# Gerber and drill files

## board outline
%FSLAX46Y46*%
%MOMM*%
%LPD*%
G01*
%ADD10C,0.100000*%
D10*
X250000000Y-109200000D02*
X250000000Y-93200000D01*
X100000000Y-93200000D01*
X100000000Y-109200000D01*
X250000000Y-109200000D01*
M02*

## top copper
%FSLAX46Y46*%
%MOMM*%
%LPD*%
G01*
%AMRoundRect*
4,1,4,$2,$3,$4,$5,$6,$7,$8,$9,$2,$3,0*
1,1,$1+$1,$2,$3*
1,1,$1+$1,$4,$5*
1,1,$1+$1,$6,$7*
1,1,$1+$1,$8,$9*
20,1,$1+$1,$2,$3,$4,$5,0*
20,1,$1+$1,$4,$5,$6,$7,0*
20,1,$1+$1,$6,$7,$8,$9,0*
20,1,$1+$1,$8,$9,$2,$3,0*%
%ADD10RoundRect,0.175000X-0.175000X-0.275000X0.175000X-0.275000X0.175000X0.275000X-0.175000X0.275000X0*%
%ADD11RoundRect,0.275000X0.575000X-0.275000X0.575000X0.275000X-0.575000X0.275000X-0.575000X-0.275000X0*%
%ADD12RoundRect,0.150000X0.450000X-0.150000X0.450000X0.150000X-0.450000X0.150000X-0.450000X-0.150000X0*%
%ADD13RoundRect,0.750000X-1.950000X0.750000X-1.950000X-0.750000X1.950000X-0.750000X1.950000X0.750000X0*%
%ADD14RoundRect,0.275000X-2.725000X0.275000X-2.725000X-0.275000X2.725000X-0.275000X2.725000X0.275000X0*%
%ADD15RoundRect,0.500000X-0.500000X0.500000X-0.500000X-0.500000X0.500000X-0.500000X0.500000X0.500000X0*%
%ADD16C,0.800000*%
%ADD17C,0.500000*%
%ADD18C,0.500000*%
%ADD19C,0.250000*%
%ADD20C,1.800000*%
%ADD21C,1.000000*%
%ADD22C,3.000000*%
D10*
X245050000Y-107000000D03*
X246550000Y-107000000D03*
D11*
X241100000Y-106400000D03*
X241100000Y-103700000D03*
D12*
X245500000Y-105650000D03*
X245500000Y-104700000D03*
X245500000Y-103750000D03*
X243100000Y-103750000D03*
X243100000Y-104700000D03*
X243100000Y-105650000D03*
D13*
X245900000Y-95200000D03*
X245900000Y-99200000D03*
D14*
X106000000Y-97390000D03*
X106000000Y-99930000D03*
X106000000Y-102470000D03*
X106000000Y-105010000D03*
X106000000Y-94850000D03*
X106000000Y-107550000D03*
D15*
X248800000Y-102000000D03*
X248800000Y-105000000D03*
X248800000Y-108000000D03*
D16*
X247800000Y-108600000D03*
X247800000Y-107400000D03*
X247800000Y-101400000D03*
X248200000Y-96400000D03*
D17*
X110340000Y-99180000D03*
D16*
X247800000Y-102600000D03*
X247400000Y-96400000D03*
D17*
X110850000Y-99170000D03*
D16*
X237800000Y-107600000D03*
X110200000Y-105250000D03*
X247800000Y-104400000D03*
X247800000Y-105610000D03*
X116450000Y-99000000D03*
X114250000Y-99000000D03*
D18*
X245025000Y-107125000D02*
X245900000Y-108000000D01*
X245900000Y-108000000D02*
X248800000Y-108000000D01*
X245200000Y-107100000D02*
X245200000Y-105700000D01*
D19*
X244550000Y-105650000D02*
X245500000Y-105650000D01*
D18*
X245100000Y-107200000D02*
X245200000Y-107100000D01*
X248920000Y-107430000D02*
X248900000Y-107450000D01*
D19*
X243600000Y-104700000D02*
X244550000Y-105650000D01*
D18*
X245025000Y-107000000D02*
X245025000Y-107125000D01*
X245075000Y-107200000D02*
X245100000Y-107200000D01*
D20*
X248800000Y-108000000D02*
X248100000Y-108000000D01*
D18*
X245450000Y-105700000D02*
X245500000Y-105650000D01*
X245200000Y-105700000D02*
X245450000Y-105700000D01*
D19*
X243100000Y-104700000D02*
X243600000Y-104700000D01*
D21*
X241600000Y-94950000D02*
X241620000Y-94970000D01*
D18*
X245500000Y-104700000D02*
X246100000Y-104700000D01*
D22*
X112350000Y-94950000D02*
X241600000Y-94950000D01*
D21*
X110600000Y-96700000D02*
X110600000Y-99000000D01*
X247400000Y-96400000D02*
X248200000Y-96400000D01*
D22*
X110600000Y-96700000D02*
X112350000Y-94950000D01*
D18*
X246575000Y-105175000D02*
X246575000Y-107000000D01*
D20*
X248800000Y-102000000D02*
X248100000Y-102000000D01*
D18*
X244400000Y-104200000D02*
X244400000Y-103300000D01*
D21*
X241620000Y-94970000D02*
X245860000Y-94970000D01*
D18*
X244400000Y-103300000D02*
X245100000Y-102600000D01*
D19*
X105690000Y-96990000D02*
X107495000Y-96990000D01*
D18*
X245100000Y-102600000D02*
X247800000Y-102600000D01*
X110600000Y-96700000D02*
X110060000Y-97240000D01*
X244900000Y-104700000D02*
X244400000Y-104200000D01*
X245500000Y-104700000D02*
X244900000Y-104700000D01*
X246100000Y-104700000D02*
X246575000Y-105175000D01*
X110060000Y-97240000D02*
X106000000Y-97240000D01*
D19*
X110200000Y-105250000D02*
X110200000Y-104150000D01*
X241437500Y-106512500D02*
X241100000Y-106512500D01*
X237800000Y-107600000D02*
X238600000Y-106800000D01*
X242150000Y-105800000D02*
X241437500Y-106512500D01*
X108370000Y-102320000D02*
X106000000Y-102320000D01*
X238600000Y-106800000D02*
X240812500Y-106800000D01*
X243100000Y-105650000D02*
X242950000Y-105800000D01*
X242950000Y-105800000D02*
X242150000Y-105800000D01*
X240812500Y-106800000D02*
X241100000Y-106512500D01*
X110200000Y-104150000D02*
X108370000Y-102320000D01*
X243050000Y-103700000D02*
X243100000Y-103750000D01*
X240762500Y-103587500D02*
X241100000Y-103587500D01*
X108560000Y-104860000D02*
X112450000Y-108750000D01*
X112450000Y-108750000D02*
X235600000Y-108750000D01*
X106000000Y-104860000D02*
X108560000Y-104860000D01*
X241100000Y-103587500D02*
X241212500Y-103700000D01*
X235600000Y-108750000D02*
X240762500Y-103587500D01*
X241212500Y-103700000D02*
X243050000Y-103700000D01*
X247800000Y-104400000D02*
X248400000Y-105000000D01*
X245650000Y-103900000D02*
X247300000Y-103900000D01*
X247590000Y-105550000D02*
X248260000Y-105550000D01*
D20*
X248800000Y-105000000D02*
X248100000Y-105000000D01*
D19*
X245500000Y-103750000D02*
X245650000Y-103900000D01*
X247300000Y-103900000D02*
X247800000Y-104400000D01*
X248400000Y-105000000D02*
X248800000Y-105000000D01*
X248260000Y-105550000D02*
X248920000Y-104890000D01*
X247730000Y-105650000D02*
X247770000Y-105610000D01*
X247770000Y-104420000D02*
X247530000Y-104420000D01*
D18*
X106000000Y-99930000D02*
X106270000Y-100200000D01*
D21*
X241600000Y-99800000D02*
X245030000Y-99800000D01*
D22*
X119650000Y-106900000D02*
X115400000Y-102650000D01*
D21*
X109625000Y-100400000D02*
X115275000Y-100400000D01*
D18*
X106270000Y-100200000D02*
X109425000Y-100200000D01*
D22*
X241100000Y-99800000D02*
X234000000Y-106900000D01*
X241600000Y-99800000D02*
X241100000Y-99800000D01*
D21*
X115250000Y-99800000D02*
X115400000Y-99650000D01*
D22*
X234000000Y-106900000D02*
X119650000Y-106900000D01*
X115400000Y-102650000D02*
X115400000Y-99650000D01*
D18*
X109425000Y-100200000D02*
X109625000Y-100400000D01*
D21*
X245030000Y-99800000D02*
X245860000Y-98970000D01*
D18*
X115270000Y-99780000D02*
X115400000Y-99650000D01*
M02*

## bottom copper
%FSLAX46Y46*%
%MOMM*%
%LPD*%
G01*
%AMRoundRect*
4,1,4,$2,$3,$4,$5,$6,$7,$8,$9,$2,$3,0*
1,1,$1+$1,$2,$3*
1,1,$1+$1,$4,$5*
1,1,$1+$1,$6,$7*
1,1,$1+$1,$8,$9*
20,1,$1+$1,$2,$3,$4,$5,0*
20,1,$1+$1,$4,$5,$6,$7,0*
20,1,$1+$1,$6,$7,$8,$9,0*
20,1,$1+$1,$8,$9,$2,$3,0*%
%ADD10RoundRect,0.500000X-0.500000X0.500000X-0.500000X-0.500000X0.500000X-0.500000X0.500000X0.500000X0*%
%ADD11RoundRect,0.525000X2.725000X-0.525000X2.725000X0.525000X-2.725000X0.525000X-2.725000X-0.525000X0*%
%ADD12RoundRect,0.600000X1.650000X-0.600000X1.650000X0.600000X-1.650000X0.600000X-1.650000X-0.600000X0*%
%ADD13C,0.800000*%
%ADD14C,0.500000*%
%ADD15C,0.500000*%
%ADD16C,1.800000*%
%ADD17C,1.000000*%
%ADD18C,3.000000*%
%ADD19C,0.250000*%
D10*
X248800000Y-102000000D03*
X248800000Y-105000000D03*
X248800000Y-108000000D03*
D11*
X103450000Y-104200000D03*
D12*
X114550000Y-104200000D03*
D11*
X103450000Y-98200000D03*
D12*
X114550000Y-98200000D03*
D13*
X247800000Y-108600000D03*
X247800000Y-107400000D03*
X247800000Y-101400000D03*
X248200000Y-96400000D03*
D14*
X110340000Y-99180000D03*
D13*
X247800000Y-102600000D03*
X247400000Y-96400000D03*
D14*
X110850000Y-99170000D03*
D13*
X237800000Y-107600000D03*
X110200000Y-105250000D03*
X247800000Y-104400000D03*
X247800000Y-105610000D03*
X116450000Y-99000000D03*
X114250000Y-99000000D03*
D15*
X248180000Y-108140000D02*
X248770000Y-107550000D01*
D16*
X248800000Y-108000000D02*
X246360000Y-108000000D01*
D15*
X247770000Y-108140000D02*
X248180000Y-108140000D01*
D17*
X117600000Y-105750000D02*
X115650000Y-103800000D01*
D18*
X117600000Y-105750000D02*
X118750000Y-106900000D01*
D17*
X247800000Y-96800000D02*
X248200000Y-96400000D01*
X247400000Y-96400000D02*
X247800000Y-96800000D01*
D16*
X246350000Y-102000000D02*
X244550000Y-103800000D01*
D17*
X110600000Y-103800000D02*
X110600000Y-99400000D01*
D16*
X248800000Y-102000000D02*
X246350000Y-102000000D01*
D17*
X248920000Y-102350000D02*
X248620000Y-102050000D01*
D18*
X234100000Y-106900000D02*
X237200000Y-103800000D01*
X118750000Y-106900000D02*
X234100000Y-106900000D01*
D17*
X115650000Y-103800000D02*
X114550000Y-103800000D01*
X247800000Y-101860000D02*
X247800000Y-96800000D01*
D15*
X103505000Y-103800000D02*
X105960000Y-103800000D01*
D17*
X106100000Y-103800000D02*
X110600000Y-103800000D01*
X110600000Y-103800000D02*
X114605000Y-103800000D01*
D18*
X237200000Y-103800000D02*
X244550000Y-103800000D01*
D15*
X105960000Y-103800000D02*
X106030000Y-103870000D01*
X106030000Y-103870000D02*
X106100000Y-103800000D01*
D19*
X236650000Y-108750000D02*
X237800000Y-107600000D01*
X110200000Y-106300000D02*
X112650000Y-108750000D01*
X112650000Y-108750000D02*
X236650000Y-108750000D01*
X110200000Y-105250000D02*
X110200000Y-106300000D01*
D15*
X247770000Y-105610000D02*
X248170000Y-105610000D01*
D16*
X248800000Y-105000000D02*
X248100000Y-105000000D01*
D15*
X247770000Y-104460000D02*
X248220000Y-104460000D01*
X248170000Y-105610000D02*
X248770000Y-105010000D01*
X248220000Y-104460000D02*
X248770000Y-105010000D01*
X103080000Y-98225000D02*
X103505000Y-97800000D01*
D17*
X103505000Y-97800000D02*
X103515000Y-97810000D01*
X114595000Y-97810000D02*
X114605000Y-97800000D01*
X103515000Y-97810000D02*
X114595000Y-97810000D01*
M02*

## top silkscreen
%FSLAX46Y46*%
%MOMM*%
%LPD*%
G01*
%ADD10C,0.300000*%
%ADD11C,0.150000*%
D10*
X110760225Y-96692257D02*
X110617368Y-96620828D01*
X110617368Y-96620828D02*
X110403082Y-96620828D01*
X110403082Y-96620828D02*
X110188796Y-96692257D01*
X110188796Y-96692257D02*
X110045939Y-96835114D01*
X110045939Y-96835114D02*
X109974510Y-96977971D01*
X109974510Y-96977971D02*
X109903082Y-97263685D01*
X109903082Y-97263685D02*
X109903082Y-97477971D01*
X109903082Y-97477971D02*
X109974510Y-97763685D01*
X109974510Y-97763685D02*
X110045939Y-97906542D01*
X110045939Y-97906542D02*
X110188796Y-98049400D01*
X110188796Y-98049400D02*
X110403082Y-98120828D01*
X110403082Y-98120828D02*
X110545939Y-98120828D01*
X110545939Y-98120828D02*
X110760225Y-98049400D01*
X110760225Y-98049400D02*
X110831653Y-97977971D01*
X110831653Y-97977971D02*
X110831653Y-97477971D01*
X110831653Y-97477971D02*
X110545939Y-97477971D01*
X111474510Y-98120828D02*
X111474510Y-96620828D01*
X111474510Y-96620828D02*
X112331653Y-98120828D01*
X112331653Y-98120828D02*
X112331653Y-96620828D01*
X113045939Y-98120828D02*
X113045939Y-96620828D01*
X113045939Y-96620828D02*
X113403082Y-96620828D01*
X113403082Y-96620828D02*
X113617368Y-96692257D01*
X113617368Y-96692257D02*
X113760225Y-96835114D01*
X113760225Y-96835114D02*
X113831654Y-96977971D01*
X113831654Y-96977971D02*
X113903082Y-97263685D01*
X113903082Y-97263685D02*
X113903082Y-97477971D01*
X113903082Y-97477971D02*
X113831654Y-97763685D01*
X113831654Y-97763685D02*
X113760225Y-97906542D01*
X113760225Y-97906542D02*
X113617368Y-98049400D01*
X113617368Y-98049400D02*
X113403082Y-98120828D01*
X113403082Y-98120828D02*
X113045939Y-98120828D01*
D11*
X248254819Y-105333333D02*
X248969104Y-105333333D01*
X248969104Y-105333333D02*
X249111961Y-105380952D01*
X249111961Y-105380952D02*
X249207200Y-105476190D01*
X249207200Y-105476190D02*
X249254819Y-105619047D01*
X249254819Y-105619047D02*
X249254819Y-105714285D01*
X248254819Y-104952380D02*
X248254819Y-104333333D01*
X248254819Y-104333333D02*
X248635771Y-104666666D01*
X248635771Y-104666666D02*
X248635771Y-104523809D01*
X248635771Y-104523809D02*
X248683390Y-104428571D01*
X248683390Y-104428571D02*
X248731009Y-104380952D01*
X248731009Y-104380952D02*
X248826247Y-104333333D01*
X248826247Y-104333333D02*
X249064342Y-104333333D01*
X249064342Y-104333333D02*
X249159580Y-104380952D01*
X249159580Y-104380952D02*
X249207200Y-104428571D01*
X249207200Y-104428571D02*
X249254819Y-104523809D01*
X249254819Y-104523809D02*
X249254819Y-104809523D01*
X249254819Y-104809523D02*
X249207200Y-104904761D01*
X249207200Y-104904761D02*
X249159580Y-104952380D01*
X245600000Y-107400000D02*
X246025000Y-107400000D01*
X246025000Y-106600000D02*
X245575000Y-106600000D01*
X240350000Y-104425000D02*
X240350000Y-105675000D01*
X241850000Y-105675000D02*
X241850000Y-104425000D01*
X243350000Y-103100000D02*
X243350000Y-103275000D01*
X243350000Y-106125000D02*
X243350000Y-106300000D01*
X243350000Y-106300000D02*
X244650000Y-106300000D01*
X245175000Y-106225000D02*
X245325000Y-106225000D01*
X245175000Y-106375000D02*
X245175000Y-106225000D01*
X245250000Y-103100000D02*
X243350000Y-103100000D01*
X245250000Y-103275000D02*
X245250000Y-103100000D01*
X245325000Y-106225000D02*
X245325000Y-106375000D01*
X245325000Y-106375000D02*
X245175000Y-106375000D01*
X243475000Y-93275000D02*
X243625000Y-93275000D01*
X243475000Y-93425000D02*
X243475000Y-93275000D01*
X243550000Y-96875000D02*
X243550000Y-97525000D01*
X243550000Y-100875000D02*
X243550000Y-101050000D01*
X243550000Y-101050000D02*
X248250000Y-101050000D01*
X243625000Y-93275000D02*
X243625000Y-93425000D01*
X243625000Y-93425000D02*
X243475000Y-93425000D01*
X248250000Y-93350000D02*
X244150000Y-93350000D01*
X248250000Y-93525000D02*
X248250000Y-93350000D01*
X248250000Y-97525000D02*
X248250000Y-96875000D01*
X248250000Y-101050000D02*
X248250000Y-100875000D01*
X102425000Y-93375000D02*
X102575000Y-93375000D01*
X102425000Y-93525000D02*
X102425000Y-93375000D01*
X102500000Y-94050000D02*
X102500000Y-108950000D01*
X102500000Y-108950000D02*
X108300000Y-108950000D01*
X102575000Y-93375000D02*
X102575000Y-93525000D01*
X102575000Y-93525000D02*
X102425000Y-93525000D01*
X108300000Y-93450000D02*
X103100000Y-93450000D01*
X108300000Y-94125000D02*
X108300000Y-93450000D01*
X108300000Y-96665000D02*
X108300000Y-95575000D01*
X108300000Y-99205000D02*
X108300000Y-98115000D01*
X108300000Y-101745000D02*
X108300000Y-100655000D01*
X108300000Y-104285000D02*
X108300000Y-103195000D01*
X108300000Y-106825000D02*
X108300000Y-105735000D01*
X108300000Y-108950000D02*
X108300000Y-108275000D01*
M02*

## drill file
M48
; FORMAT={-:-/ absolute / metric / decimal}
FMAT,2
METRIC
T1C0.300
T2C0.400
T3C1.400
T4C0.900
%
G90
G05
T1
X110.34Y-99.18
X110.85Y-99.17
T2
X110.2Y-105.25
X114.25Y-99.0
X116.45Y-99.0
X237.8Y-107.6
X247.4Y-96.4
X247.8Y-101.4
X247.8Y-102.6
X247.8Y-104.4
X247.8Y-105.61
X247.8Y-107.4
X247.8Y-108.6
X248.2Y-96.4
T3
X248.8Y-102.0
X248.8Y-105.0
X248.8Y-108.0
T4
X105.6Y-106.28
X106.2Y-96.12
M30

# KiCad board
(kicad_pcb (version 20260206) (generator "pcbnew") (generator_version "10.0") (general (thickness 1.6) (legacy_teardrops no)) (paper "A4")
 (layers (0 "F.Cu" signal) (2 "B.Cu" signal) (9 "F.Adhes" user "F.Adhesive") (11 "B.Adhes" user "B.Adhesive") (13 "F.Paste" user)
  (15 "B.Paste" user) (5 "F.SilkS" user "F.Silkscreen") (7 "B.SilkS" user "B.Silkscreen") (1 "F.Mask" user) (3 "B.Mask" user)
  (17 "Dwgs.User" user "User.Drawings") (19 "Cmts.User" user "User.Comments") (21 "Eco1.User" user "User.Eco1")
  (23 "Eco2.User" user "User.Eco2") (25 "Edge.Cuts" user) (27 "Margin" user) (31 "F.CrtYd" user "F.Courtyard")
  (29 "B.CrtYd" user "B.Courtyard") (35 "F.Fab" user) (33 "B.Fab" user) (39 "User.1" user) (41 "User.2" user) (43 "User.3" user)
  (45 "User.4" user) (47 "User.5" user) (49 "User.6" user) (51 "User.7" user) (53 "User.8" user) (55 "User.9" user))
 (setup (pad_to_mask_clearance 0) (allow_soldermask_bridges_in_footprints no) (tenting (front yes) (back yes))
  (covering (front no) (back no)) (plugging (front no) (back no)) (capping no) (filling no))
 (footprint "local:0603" (layer "F.Cu") (at 245.8 107)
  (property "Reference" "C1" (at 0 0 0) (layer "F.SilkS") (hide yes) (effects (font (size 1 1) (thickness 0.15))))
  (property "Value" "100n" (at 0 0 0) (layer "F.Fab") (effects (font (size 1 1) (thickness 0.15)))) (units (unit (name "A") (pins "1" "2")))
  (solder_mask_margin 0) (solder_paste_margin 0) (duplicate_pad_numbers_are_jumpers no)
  (fp_line (start -0.2 0.4) (end 0.225 0.4) (stroke (width 0.15) (type solid)) (layer "F.SilkS"))
  (fp_line (start 0.225 -0.4) (end -0.225 -0.4) (stroke (width 0.15) (type solid)) (layer "F.SilkS"))
  (pad "1" smd roundrect (at -0.75 0) (size 0.7 0.9) (layers "F.Cu" "F.Mask" "F.Paste") (roundrect_rratio 0.25) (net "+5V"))
  (pad "2" smd roundrect (at 0.75 0) (size 0.7 0.9) (layers "F.Cu" "F.Mask" "F.Paste") (roundrect_rratio 0.25) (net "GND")))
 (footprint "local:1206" (layer "F.Cu") (at 241.1 105.05 90)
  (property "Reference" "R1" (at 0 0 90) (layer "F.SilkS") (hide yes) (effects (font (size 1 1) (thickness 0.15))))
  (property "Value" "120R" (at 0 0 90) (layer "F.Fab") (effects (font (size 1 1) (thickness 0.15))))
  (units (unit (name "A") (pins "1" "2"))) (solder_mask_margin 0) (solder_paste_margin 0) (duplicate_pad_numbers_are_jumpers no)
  (fp_line (start 0.625 -0.75) (end -0.625 -0.75) (stroke (width 0.15) (type solid)) (layer "F.SilkS"))
  (fp_line (start -0.625 0.75) (end 0.625 0.75) (stroke (width 0.15) (type solid)) (layer "F.SilkS"))
  (pad "1" smd roundrect (at -1.35 0 90) (size 1.1 1.7) (layers "F.Cu" "F.Mask" "F.Paste") (roundrect_rratio 0.25) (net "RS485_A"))
  (pad "2" smd roundrect (at 1.35 0 90) (size 1.1 1.7) (layers "F.Cu" "F.Mask" "F.Paste") (roundrect_rratio 0.25) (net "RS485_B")))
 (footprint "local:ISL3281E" (layer "F.Cu") (at 244.3 104.7 90)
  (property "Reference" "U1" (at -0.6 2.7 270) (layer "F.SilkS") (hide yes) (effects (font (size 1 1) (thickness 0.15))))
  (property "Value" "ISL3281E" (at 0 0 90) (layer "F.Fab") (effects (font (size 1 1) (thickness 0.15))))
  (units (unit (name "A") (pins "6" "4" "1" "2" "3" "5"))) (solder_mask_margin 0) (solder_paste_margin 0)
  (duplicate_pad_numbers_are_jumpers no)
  (fp_line (start 1.6 -0.95) (end 1.425 -0.95) (stroke (width 0.15) (type solid)) (layer "F.SilkS"))
  (fp_line (start -1.425 -0.95) (end -1.6 -0.95) (stroke (width 0.15) (type solid)) (layer "F.SilkS"))
  (fp_line (start -1.6 -0.95) (end -1.6 0.35) (stroke (width 0.15) (type solid)) (layer "F.SilkS"))
  (fp_line (start -1.525 0.875) (end -1.525 1.025) (stroke (width 0.15) (type solid)) (layer "F.SilkS"))
  (fp_line (start -1.675 0.875) (end -1.525 0.875) (stroke (width 0.15) (type solid)) (layer "F.SilkS"))
  (fp_line (start 1.6 0.95) (end 1.6 -0.95) (stroke (width 0.15) (type solid)) (layer "F.SilkS"))
  (fp_line (start 1.425 0.95) (end 1.6 0.95) (stroke (width 0.15) (type solid)) (layer "F.SilkS"))
  (fp_line (start -1.525 1.025) (end -1.675 1.025) (stroke (width 0.15) (type solid)) (layer "F.SilkS"))
  (fp_line (start -1.675 1.025) (end -1.675 0.875) (stroke (width 0.15) (type solid)) (layer "F.SilkS"))
  (pad "1" smd roundrect (at -0.95 1.2 90) (size 0.6 1.2) (layers "F.Cu" "F.Mask" "F.Paste") (roundrect_rratio 0.25) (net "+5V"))
  (pad "2" smd roundrect (at 0 1.2 90) (size 0.6 1.2) (layers "F.Cu" "F.Mask" "F.Paste") (roundrect_rratio 0.25) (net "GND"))
  (pad "3" smd roundrect (at 0.95 1.2 90) (size 0.6 1.2) (layers "F.Cu" "F.Mask" "F.Paste") (roundrect_rratio 0.25) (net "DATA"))
  (pad "4" smd roundrect (at 0.95 -1.2 90) (size 0.6 1.2) (layers "F.Cu" "F.Mask" "F.Paste") (roundrect_rratio 0.25) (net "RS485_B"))
  (pad "5" smd roundrect (at 0 -1.2 90) (size 0.6 1.2) (layers "F.Cu" "F.Mask" "F.Paste") (roundrect_rratio 0.25) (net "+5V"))
  (pad "6" smd roundrect (at -0.95 -1.2 90) (size 0.6 1.2) (layers "F.Cu" "F.Mask" "F.Paste") (roundrect_rratio 0.25) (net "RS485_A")))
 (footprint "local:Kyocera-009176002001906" (layer "F.Cu") (at 245.9 97.2 -90)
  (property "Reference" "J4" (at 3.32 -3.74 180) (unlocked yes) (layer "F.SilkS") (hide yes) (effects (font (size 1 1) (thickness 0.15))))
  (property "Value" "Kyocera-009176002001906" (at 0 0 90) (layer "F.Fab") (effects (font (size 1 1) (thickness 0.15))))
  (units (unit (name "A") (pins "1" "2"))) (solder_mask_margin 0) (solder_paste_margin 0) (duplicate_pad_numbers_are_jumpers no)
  (fp_line (start -3.925 2.425) (end -3.925 2.275) (stroke (width 0.15) (type solid)) (layer "F.SilkS"))
  (fp_line (start -3.775 2.425) (end -3.925 2.425) (stroke (width 0.15) (type solid)) (layer "F.SilkS"))
  (fp_line (start -0.325 2.35) (end 0.325 2.35) (stroke (width 0.15) (type solid)) (layer "F.SilkS"))
  (fp_line (start 3.675 2.35) (end 3.85 2.35) (stroke (width 0.15) (type solid)) (layer "F.SilkS"))
  (fp_line (start 3.85 2.35) (end 3.85 -2.35) (stroke (width 0.15) (type solid)) (layer "F.SilkS"))
  (fp_line (start -3.925 2.275) (end -3.775 2.275) (stroke (width 0.15) (type solid)) (layer "F.SilkS"))
  (fp_line (start -3.775 2.275) (end -3.775 2.425) (stroke (width 0.15) (type solid)) (layer "F.SilkS"))
  (fp_line (start -3.85 -2.35) (end -3.85 1.75) (stroke (width 0.15) (type solid)) (layer "F.SilkS"))
  (fp_line (start -3.675 -2.35) (end -3.85 -2.35) (stroke (width 0.15) (type solid)) (layer "F.SilkS"))
  (fp_line (start 0.325 -2.35) (end -0.325 -2.35) (stroke (width 0.15) (type solid)) (layer "F.SilkS"))
  (fp_line (start 3.85 -2.35) (end 3.675 -2.35) (stroke (width 0.15) (type solid)) (layer "F.SilkS"))
  (pad "1" smd roundrect (at -2 0 270) (size 3 5.4) (layers "F.Cu" "F.Mask" "F.Paste") (roundrect_rratio 0.25) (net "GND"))
  (pad "2" smd roundrect (at 2 0 270) (size 3 5.4) (layers "F.Cu" "F.Mask" "F.Paste") (roundrect_rratio 0.25) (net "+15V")))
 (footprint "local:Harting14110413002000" (layer "F.Cu") (at 106 101.2 -90)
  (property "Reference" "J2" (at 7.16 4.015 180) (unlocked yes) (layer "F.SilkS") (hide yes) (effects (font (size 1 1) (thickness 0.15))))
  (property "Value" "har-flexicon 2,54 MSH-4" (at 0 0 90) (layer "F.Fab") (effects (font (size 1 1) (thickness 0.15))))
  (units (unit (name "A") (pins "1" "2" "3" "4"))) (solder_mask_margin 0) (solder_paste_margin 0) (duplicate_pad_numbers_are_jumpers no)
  (fp_line (start -7.825 3.575) (end -7.825 3.425) (stroke (width 0.15) (type solid)) (layer "F.SilkS"))
  (fp_line (start -7.675 3.575) (end -7.825 3.575) (stroke (width 0.15) (type solid)) (layer "F.SilkS"))
  (fp_line (start -7.15 3.5) (end 7.75 3.5) (stroke (width 0.15) (type solid)) (layer "F.SilkS"))
  (fp_line (start 7.75 3.5) (end 7.75 -2.3) (stroke (width 0.15) (type solid)) (layer "F.SilkS"))
  (fp_line (start -7.825 3.425) (end -7.675 3.425) (stroke (width 0.15) (type solid)) (layer "F.SilkS"))
  (fp_line (start -7.675 3.425) (end -7.675 3.575) (stroke (width 0.15) (type solid)) (layer "F.SilkS"))
  (fp_line (start -7.75 -2.3) (end -7.75 2.9) (stroke (width 0.15) (type solid)) (layer "F.SilkS"))
  (fp_line (start -7.075 -2.3) (end -7.75 -2.3) (stroke (width 0.15) (type solid)) (layer "F.SilkS"))
  (fp_line (start -4.535 -2.3) (end -5.625 -2.3) (stroke (width 0.15) (type solid)) (layer "F.SilkS"))
  (fp_line (start -1.995 -2.3) (end -3.085 -2.3) (stroke (width 0.15) (type solid)) (layer "F.SilkS"))
  (fp_line (start 0.545 -2.3) (end -0.545 -2.3) (stroke (width 0.15) (type solid)) (layer "F.SilkS"))
  (fp_line (start 3.085 -2.3) (end 1.995 -2.3) (stroke (width 0.15) (type solid)) (layer "F.SilkS"))
  (fp_line (start 5.625 -2.3) (end 4.535 -2.3) (stroke (width 0.15) (type solid)) (layer "F.SilkS"))
  (fp_line (start 7.75 -2.3) (end 7.075 -2.3) (stroke (width 0.15) (type solid)) (layer "F.SilkS"))
  (pad "" np_thru_hole circle (at -5.08 -0.2 270) (size 0.9 0.9) (drill 0.9) (layers "*.Cu" "*.Mask"))
  (pad "" np_thru_hole circle (at 5.08 0.4 270) (size 0.9 0.9) (drill 0.9) (layers "*.Cu" "*.Mask"))
  (pad "1" smd roundrect (at -3.81 0 270) (size 1.1 6) (layers "F.Cu" "F.Mask" "F.Paste") (roundrect_rratio 0.25) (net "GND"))
  (pad "2" smd roundrect (at -1.27 0 270) (size 1.1 6) (layers "F.Cu" "F.Mask" "F.Paste") (roundrect_rratio 0.25) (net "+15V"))
  (pad "3" smd roundrect (at 1.27 0 270) (size 1.1 6) (layers "F.Cu" "F.Mask" "F.Paste") (roundrect_rratio 0.25) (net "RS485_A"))
  (pad "4" smd roundrect (at 3.81 0 270) (size 1.1 6) (layers "F.Cu" "F.Mask" "F.Paste") (roundrect_rratio 0.25) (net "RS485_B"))
  (pad "MP1" smd roundrect (at -6.35 0 270) (size 1.1 6) (layers "F.Cu" "F.Mask" "F.Paste") (roundrect_rratio 0.25))
  (pad "MP2" smd roundrect (at 6.35 0 270) (size 1.1 6) (layers "F.Cu" "F.Mask" "F.Paste") (roundrect_rratio 0.25)))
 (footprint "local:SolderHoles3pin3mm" (layer "F.Cu") (at 248.8 105 -90)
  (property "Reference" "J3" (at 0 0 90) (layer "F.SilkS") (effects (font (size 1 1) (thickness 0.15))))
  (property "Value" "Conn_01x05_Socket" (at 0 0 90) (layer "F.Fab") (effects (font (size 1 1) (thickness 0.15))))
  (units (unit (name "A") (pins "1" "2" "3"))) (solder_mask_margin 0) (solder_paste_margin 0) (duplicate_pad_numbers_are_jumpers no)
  (pad "1" thru_hole roundrect (at -3 0 270) (size 2 2) (drill 1.4) (layers "*.Cu" "*.Mask") (remove_unused_layers yes)
   (keep_end_layers yes) (zone_layer_connections) (roundrect_rratio 0.25) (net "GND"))
  (pad "2" thru_hole roundrect (at 0 0 270) (size 2 2) (drill 1.4) (layers "*.Cu" "*.Mask") (remove_unused_layers yes) (keep_end_layers yes)
   (zone_layer_connections) (roundrect_rratio 0.25) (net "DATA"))
  (pad "3" thru_hole roundrect (at 3 0 270) (size 2 2) (drill 1.4) (layers "*.Cu" "*.Mask") (remove_unused_layers yes) (keep_end_layers yes)
   (zone_layer_connections) (roundrect_rratio 0.25) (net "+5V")))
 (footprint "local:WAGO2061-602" (layer "B.Cu") (at 108.2 101.2 90)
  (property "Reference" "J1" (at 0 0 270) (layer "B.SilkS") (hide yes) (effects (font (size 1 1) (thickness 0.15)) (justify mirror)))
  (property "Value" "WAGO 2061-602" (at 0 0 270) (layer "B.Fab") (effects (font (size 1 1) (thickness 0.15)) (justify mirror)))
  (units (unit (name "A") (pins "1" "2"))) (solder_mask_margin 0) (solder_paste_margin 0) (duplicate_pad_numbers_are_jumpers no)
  (pad "1" smd roundrect (at -3 -4.75 90) (size 2.1 6.5) (layers "B.Cu" "B.Mask" "B.Paste") (roundrect_rratio 0.25) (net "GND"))
  (pad "1" smd roundrect (at -3 6.35 90) (size 2.4 4.5) (layers "B.Cu" "B.Mask" "B.Paste") (roundrect_rratio 0.25) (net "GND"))
  (pad "2" smd roundrect (at 3 -4.75 90) (size 2.1 6.5) (layers "B.Cu" "B.Mask" "B.Paste") (roundrect_rratio 0.25) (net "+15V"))
  (pad "2" smd roundrect (at 3 6.35 90) (size 2.4 4.5) (layers "B.Cu" "B.Mask" "B.Paste") (roundrect_rratio 0.25) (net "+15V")))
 (gr_poly (pts (xy 250 109.2) (xy 250 93.2) (xy 100 93.2) (xy 100 109.2)) (stroke (width 0.1) (type solid)) (fill no) (layer "Edge.Cuts"))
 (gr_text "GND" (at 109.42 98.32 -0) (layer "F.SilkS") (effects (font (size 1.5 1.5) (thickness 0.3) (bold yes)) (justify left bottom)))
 (segment (start 245.025 107.125) (end 245.9 108) (width 0.5) (layer "F.Cu") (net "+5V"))
 (segment (start 245.9 108) (end 248.8 108) (width 0.5) (layer "F.Cu") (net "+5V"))
 (segment (start 245.2 107.1) (end 245.2 105.7) (width 0.5) (layer "F.Cu") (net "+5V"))
 (segment (start 244.55 105.65) (end 245.5 105.65) (width 0.25) (layer "F.Cu") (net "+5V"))
 (segment (start 245.1 107.2) (end 245.2 107.1) (width 0.5) (layer "F.Cu") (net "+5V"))
 (segment (start 248.92 107.43) (end 248.9 107.45) (width 0.5) (layer "F.Cu") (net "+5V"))
 (segment (start 243.6 104.7) (end 244.55 105.65) (width 0.25) (layer "F.Cu") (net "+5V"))
 (segment (start 245.025 107) (end 245.025 107.125) (width 0.5) (layer "F.Cu") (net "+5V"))
 (segment (start 245.075 107.2) (end 245.1 107.2) (width 0.5) (layer "F.Cu") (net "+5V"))
 (segment (start 248.8 108) (end 248.1 108) (width 1.8) (layer "F.Cu") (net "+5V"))
 (segment (start 245.45 105.7) (end 245.5 105.65) (width 0.5) (layer "F.Cu") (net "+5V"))
 (segment (start 245.2 105.7) (end 245.45 105.7) (width 0.5) (layer "F.Cu") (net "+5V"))
 (segment (start 243.1 104.7) (end 243.6 104.7) (width 0.25) (layer "F.Cu") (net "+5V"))
 (via (at 247.8 108.6) (size 0.8) (drill 0.4) (layers "F.Cu" "B.Cu") (capping no) (covering (front no) (back no))
  (plugging (front no) (back no)) (filling no) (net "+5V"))
 (via (at 247.8 107.4) (size 0.8) (drill 0.4) (layers "F.Cu" "B.Cu") (capping no) (covering (front no) (back no))
  (plugging (front no) (back no)) (filling no) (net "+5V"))
 (segment (start 248.18 108.14) (end 248.77 107.55) (width 0.5) (layer "B.Cu") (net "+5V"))
 (segment (start 248.8 108) (end 246.36 108) (width 1.8) (layer "B.Cu") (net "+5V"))
 (segment (start 247.77 108.14) (end 248.18 108.14) (width 0.5) (layer "B.Cu") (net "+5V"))
 (segment (start 241.6 94.95) (end 241.62 94.97) (width 1) (layer "F.Cu") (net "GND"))
 (segment (start 245.5 104.7) (end 246.1 104.7) (width 0.5) (layer "F.Cu") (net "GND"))
 (segment (start 112.35 94.95) (end 241.6 94.95) (width 3) (layer "F.Cu") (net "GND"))
 (segment (start 110.6 96.7) (end 110.6 99) (width 1) (layer "F.Cu") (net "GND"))
 (segment (start 247.4 96.4) (end 248.2 96.4) (width 1) (layer "F.Cu") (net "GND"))
 (segment (start 110.6 96.7) (end 112.35 94.95) (width 3) (layer "F.Cu") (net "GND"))
 (segment (start 246.575 105.175) (end 246.575 107) (width 0.5) (layer "F.Cu") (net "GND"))
 (segment (start 248.8 102) (end 248.1 102) (width 1.8) (layer "F.Cu") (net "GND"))
 (segment (start 244.4 104.2) (end 244.4 103.3) (width 0.5) (layer "F.Cu") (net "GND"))
 (segment (start 241.62 94.97) (end 245.86 94.97) (width 1) (layer "F.Cu") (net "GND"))
 (segment (start 244.4 103.3) (end 245.1 102.6) (width 0.5) (layer "F.Cu") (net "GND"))
 (segment (start 105.69 96.99) (end 107.495 96.99) (width 0.25) (layer "F.Cu") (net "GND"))
 (segment (start 245.1 102.6) (end 247.8 102.6) (width 0.5) (layer "F.Cu") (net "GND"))
 (segment (start 110.6 96.7) (end 110.06 97.24) (width 0.5) (layer "F.Cu") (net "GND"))
 (segment (start 244.9 104.7) (end 244.4 104.2) (width 0.5) (layer "F.Cu") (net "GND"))
 (segment (start 245.5 104.7) (end 244.9 104.7) (width 0.5) (layer "F.Cu") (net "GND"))
 (segment (start 246.1 104.7) (end 246.575 105.175) (width 0.5) (layer "F.Cu") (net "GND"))
 (segment (start 110.06 97.24) (end 106 97.24) (width 0.5) (layer "F.Cu") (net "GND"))
 (via (at 247.8 101.4) (size 0.8) (drill 0.4) (layers "F.Cu" "B.Cu") (capping no) (covering (front no) (back no))
  (plugging (front no) (back no)) (filling no) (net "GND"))
 (via (at 248.2 96.4) (size 0.8) (drill 0.4) (layers "F.Cu" "B.Cu") (capping no) (covering (front no) (back no))
  (plugging (front no) (back no)) (filling no) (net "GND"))
 (via (at 110.34 99.18) (size 0.5) (drill 0.3) (layers "F.Cu" "B.Cu") (capping no) (covering (front no) (back no))
  (plugging (front no) (back no)) (filling no) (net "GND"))
 (via (at 247.8 102.6) (size 0.8) (drill 0.4) (layers "F.Cu" "B.Cu") (capping no) (covering (front no) (back no))
  (plugging (front no) (back no)) (filling no) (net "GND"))
 (via (at 247.4 96.4) (size 0.8) (drill 0.4) (layers "F.Cu" "B.Cu") (capping no) (covering (front no) (back no))
  (plugging (front no) (back no)) (filling no) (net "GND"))
 (via (at 110.85 99.17) (size 0.5) (drill 0.3) (layers "F.Cu" "B.Cu") (capping no) (covering (front no) (back no))
  (plugging (front no) (back no)) (filling no) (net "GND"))
 (segment (start 117.6 105.75) (end 115.65 103.8) (width 1) (layer "B.Cu") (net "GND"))
 (segment (start 117.6 105.75) (end 118.75 106.9) (width 3) (layer "B.Cu") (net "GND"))
 (segment (start 247.8 96.8) (end 248.2 96.4) (width 1) (layer "B.Cu") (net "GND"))
 (segment (start 247.4 96.4) (end 247.8 96.8) (width 1) (layer "B.Cu") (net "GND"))
 (segment (start 246.35 102) (end 244.55 103.8) (width 1.8) (layer "B.Cu") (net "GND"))
 (segment (start 110.6 103.8) (end 110.6 99.4) (width 1) (layer "B.Cu") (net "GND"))
 (segment (start 248.8 102) (end 246.35 102) (width 1.8) (layer "B.Cu") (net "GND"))
 (segment (start 248.92 102.35) (end 248.62 102.05) (width 1) (layer "B.Cu") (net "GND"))
 (segment (start 234.1 106.9) (end 237.2 103.8) (width 3) (layer "B.Cu") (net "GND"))
 (segment (start 118.75 106.9) (end 234.1 106.9) (width 3) (layer "B.Cu") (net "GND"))
 (segment (start 115.65 103.8) (end 114.55 103.8) (width 1) (layer "B.Cu") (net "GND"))
 (segment (start 247.8 101.86) (end 247.8 96.8) (width 1) (layer "B.Cu") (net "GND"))
 (segment (start 103.505 103.8) (end 105.96 103.8) (width 0.5) (layer "B.Cu") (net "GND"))
 (segment (start 106.1 103.8) (end 110.6 103.8) (width 1) (layer "B.Cu") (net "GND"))
 (segment (start 110.6 103.8) (end 114.605 103.8) (width 1) (layer "B.Cu") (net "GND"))
 (segment (start 237.2 103.8) (end 244.55 103.8) (width 3) (layer "B.Cu") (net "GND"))
 (segment (start 105.96 103.8) (end 106.03 103.87) (width 0.5) (layer "B.Cu") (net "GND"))
 (segment (start 106.03 103.87) (end 106.1 103.8) (width 0.5) (layer "B.Cu") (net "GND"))
 (segment (start 110.2 105.25) (end 110.2 104.15) (width 0.25) (layer "F.Cu") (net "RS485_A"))
 (segment (start 241.4375 106.5125) (end 241.1 106.5125) (width 0.25) (layer "F.Cu") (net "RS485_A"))
 (segment (start 237.8 107.6) (end 238.6 106.8) (width 0.25) (layer "F.Cu") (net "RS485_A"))
 (segment (start 242.15 105.8) (end 241.4375 106.5125) (width 0.25) (layer "F.Cu") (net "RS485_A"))
 (segment (start 108.37 102.32) (end 106 102.32) (width 0.25) (layer "F.Cu") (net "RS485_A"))
 (segment (start 238.6 106.8) (end 240.8125 106.8) (width 0.25) (layer "F.Cu") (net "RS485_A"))
 (segment (start 243.1 105.65) (end 242.95 105.8) (width 0.25) (layer "F.Cu") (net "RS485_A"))
 (segment (start 242.95 105.8) (end 242.15 105.8) (width 0.25) (layer "F.Cu") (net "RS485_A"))
 (segment (start 240.8125 106.8) (end 241.1 106.5125) (width 0.25) (layer "F.Cu") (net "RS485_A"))
 (segment (start 110.2 104.15) (end 108.37 102.32) (width 0.25) (layer "F.Cu") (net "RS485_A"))
 (via (at 237.8 107.6) (size 0.8) (drill 0.4) (layers "F.Cu" "B.Cu") (capping no) (covering (front no) (back no))
  (plugging (front no) (back no)) (filling no) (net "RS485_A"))
 (via (at 110.2 105.25) (size 0.8) (drill 0.4) (layers "F.Cu" "B.Cu") (capping no) (covering (front no) (back no))
  (plugging (front no) (back no)) (filling no) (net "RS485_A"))
 (segment (start 236.65 108.75) (end 237.8 107.6) (width 0.25) (layer "B.Cu") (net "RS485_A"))
 (segment (start 110.2 106.3) (end 112.65 108.75) (width 0.25) (layer "B.Cu") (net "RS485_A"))
 (segment (start 112.65 108.75) (end 236.65 108.75) (width 0.25) (layer "B.Cu") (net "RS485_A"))
 (segment (start 110.2 105.25) (end 110.2 106.3) (width 0.25) (layer "B.Cu") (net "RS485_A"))
 (segment (start 243.05 103.7) (end 243.1 103.75) (width 0.25) (layer "F.Cu") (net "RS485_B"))
 (segment (start 240.7625 103.5875) (end 241.1 103.5875) (width 0.25) (layer "F.Cu") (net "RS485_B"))
 (segment (start 108.56 104.86) (end 112.45 108.75) (width 0.25) (layer "F.Cu") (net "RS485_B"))
 (segment (start 112.45 108.75) (end 235.6 108.75) (width 0.25) (layer "F.Cu") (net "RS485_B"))
 (segment (start 106 104.86) (end 108.56 104.86) (width 0.25) (layer "F.Cu") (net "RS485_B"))
 (segment (start 241.1 103.5875) (end 241.2125 103.7) (width 0.25) (layer "F.Cu") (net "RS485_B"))
 (segment (start 235.6 108.75) (end 240.7625 103.5875) (width 0.25) (layer "F.Cu") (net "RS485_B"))
 (segment (start 241.2125 103.7) (end 243.05 103.7) (width 0.25) (layer "F.Cu") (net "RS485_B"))
 (segment (start 247.8 104.4) (end 248.4 105) (width 0.25) (layer "F.Cu") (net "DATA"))
 (segment (start 245.65 103.9) (end 247.3 103.9) (width 0.25) (layer "F.Cu") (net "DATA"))
 (segment (start 247.59 105.55) (end 248.26 105.55) (width 0.25) (layer "F.Cu") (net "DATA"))
 (segment (start 248.8 105) (end 248.1 105) (width 1.8) (layer "F.Cu") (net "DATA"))
 (segment (start 245.5 103.75) (end 245.65 103.9) (width 0.25) (layer "F.Cu") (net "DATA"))
 (segment (start 247.3 103.9) (end 247.8 104.4) (width 0.25) (layer "F.Cu") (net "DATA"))
 (segment (start 248.4 105) (end 248.8 105) (width 0.25) (layer "F.Cu") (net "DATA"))
 (segment (start 248.26 105.55) (end 248.92 104.89) (width 0.25) (layer "F.Cu") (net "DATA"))
 (segment (start 247.73 105.65) (end 247.77 105.61) (width 0.25) (layer "F.Cu") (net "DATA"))
 (segment (start 247.77 104.42) (end 247.53 104.42) (width 0.25) (layer "F.Cu") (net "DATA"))
 (via (at 247.8 104.4) (size 0.8) (drill 0.4) (layers "F.Cu" "B.Cu") (capping no) (covering (front no) (back no))
  (plugging (front no) (back no)) (filling no) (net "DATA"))
 (via (at 247.8 105.61) (size 0.8) (drill 0.4) (layers "F.Cu" "B.Cu") (capping no) (covering (front no) (back no))
  (plugging (front no) (back no)) (filling no) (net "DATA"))
 (segment (start 247.77 105.61) (end 248.17 105.61) (width 0.5) (layer "B.Cu") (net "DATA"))
 (segment (start 248.8 105) (end 248.1 105) (width 1.8) (layer "B.Cu") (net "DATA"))
 (segment (start 247.77 104.46) (end 248.22 104.46) (width 0.5) (layer "B.Cu") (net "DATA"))
 (segment (start 248.17 105.61) (end 248.77 105.01) (width 0.5) (layer "B.Cu") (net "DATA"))
 (segment (start 248.22 104.46) (end 248.77 105.01) (width 0.5) (layer "B.Cu") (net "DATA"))
 (segment (start 106 99.93) (end 106.27 100.2) (width 0.5) (layer "F.Cu") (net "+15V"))
 (segment (start 241.6 99.8) (end 245.03 99.8) (width 1) (layer "F.Cu") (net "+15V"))
 (segment (start 119.65 106.9) (end 115.4 102.65) (width 3) (layer "F.Cu") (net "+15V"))
 (segment (start 109.625 100.4) (end 115.275 100.4) (width 1) (layer "F.Cu") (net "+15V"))
 (segment (start 106.27 100.2) (end 109.425 100.2) (width 0.5) (layer "F.Cu") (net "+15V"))
 (segment (start 241.1 99.8) (end 234 106.9) (width 3) (layer "F.Cu") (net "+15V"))
 (segment (start 241.6 99.8) (end 241.1 99.8) (width 3) (layer "F.Cu") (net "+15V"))
 (segment (start 115.25 99.8) (end 115.4 99.65) (width 1) (layer "F.Cu") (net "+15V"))
 (segment (start 234 106.9) (end 119.65 106.9) (width 3) (layer "F.Cu") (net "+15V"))
 (segment (start 115.4 102.65) (end 115.4 99.65) (width 3) (layer "F.Cu") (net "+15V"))
 (segment (start 109.425 100.2) (end 109.625 100.4) (width 0.5) (layer "F.Cu") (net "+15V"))
 (segment (start 245.03 99.8) (end 245.86 98.97) (width 1) (layer "F.Cu") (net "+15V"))
 (segment (start 115.27 99.78) (end 115.4 99.65) (width 0.5) (layer "F.Cu") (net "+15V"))
 (via (at 116.45 99) (size 0.8) (drill 0.4) (layers "F.Cu" "B.Cu") (capping no) (covering (front no) (back no))
  (plugging (front no) (back no)) (filling no) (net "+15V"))
 (via (at 114.25 99) (size 0.8) (drill 0.4) (layers "F.Cu" "B.Cu") (capping no) (covering (front no) (back no))
  (plugging (front no) (back no)) (filling no) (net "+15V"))
 (segment (start 103.08 98.225) (end 103.505 97.8) (width 0.5) (layer "B.Cu") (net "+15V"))
 (segment (start 103.505 97.8) (end 103.515 97.81) (width 1) (layer "B.Cu") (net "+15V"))
 (segment (start 114.595 97.81) (end 114.605 97.8) (width 1) (layer "B.Cu") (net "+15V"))
 (segment (start 103.515 97.81) (end 114.595 97.81) (width 1) (layer "B.Cu") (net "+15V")))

